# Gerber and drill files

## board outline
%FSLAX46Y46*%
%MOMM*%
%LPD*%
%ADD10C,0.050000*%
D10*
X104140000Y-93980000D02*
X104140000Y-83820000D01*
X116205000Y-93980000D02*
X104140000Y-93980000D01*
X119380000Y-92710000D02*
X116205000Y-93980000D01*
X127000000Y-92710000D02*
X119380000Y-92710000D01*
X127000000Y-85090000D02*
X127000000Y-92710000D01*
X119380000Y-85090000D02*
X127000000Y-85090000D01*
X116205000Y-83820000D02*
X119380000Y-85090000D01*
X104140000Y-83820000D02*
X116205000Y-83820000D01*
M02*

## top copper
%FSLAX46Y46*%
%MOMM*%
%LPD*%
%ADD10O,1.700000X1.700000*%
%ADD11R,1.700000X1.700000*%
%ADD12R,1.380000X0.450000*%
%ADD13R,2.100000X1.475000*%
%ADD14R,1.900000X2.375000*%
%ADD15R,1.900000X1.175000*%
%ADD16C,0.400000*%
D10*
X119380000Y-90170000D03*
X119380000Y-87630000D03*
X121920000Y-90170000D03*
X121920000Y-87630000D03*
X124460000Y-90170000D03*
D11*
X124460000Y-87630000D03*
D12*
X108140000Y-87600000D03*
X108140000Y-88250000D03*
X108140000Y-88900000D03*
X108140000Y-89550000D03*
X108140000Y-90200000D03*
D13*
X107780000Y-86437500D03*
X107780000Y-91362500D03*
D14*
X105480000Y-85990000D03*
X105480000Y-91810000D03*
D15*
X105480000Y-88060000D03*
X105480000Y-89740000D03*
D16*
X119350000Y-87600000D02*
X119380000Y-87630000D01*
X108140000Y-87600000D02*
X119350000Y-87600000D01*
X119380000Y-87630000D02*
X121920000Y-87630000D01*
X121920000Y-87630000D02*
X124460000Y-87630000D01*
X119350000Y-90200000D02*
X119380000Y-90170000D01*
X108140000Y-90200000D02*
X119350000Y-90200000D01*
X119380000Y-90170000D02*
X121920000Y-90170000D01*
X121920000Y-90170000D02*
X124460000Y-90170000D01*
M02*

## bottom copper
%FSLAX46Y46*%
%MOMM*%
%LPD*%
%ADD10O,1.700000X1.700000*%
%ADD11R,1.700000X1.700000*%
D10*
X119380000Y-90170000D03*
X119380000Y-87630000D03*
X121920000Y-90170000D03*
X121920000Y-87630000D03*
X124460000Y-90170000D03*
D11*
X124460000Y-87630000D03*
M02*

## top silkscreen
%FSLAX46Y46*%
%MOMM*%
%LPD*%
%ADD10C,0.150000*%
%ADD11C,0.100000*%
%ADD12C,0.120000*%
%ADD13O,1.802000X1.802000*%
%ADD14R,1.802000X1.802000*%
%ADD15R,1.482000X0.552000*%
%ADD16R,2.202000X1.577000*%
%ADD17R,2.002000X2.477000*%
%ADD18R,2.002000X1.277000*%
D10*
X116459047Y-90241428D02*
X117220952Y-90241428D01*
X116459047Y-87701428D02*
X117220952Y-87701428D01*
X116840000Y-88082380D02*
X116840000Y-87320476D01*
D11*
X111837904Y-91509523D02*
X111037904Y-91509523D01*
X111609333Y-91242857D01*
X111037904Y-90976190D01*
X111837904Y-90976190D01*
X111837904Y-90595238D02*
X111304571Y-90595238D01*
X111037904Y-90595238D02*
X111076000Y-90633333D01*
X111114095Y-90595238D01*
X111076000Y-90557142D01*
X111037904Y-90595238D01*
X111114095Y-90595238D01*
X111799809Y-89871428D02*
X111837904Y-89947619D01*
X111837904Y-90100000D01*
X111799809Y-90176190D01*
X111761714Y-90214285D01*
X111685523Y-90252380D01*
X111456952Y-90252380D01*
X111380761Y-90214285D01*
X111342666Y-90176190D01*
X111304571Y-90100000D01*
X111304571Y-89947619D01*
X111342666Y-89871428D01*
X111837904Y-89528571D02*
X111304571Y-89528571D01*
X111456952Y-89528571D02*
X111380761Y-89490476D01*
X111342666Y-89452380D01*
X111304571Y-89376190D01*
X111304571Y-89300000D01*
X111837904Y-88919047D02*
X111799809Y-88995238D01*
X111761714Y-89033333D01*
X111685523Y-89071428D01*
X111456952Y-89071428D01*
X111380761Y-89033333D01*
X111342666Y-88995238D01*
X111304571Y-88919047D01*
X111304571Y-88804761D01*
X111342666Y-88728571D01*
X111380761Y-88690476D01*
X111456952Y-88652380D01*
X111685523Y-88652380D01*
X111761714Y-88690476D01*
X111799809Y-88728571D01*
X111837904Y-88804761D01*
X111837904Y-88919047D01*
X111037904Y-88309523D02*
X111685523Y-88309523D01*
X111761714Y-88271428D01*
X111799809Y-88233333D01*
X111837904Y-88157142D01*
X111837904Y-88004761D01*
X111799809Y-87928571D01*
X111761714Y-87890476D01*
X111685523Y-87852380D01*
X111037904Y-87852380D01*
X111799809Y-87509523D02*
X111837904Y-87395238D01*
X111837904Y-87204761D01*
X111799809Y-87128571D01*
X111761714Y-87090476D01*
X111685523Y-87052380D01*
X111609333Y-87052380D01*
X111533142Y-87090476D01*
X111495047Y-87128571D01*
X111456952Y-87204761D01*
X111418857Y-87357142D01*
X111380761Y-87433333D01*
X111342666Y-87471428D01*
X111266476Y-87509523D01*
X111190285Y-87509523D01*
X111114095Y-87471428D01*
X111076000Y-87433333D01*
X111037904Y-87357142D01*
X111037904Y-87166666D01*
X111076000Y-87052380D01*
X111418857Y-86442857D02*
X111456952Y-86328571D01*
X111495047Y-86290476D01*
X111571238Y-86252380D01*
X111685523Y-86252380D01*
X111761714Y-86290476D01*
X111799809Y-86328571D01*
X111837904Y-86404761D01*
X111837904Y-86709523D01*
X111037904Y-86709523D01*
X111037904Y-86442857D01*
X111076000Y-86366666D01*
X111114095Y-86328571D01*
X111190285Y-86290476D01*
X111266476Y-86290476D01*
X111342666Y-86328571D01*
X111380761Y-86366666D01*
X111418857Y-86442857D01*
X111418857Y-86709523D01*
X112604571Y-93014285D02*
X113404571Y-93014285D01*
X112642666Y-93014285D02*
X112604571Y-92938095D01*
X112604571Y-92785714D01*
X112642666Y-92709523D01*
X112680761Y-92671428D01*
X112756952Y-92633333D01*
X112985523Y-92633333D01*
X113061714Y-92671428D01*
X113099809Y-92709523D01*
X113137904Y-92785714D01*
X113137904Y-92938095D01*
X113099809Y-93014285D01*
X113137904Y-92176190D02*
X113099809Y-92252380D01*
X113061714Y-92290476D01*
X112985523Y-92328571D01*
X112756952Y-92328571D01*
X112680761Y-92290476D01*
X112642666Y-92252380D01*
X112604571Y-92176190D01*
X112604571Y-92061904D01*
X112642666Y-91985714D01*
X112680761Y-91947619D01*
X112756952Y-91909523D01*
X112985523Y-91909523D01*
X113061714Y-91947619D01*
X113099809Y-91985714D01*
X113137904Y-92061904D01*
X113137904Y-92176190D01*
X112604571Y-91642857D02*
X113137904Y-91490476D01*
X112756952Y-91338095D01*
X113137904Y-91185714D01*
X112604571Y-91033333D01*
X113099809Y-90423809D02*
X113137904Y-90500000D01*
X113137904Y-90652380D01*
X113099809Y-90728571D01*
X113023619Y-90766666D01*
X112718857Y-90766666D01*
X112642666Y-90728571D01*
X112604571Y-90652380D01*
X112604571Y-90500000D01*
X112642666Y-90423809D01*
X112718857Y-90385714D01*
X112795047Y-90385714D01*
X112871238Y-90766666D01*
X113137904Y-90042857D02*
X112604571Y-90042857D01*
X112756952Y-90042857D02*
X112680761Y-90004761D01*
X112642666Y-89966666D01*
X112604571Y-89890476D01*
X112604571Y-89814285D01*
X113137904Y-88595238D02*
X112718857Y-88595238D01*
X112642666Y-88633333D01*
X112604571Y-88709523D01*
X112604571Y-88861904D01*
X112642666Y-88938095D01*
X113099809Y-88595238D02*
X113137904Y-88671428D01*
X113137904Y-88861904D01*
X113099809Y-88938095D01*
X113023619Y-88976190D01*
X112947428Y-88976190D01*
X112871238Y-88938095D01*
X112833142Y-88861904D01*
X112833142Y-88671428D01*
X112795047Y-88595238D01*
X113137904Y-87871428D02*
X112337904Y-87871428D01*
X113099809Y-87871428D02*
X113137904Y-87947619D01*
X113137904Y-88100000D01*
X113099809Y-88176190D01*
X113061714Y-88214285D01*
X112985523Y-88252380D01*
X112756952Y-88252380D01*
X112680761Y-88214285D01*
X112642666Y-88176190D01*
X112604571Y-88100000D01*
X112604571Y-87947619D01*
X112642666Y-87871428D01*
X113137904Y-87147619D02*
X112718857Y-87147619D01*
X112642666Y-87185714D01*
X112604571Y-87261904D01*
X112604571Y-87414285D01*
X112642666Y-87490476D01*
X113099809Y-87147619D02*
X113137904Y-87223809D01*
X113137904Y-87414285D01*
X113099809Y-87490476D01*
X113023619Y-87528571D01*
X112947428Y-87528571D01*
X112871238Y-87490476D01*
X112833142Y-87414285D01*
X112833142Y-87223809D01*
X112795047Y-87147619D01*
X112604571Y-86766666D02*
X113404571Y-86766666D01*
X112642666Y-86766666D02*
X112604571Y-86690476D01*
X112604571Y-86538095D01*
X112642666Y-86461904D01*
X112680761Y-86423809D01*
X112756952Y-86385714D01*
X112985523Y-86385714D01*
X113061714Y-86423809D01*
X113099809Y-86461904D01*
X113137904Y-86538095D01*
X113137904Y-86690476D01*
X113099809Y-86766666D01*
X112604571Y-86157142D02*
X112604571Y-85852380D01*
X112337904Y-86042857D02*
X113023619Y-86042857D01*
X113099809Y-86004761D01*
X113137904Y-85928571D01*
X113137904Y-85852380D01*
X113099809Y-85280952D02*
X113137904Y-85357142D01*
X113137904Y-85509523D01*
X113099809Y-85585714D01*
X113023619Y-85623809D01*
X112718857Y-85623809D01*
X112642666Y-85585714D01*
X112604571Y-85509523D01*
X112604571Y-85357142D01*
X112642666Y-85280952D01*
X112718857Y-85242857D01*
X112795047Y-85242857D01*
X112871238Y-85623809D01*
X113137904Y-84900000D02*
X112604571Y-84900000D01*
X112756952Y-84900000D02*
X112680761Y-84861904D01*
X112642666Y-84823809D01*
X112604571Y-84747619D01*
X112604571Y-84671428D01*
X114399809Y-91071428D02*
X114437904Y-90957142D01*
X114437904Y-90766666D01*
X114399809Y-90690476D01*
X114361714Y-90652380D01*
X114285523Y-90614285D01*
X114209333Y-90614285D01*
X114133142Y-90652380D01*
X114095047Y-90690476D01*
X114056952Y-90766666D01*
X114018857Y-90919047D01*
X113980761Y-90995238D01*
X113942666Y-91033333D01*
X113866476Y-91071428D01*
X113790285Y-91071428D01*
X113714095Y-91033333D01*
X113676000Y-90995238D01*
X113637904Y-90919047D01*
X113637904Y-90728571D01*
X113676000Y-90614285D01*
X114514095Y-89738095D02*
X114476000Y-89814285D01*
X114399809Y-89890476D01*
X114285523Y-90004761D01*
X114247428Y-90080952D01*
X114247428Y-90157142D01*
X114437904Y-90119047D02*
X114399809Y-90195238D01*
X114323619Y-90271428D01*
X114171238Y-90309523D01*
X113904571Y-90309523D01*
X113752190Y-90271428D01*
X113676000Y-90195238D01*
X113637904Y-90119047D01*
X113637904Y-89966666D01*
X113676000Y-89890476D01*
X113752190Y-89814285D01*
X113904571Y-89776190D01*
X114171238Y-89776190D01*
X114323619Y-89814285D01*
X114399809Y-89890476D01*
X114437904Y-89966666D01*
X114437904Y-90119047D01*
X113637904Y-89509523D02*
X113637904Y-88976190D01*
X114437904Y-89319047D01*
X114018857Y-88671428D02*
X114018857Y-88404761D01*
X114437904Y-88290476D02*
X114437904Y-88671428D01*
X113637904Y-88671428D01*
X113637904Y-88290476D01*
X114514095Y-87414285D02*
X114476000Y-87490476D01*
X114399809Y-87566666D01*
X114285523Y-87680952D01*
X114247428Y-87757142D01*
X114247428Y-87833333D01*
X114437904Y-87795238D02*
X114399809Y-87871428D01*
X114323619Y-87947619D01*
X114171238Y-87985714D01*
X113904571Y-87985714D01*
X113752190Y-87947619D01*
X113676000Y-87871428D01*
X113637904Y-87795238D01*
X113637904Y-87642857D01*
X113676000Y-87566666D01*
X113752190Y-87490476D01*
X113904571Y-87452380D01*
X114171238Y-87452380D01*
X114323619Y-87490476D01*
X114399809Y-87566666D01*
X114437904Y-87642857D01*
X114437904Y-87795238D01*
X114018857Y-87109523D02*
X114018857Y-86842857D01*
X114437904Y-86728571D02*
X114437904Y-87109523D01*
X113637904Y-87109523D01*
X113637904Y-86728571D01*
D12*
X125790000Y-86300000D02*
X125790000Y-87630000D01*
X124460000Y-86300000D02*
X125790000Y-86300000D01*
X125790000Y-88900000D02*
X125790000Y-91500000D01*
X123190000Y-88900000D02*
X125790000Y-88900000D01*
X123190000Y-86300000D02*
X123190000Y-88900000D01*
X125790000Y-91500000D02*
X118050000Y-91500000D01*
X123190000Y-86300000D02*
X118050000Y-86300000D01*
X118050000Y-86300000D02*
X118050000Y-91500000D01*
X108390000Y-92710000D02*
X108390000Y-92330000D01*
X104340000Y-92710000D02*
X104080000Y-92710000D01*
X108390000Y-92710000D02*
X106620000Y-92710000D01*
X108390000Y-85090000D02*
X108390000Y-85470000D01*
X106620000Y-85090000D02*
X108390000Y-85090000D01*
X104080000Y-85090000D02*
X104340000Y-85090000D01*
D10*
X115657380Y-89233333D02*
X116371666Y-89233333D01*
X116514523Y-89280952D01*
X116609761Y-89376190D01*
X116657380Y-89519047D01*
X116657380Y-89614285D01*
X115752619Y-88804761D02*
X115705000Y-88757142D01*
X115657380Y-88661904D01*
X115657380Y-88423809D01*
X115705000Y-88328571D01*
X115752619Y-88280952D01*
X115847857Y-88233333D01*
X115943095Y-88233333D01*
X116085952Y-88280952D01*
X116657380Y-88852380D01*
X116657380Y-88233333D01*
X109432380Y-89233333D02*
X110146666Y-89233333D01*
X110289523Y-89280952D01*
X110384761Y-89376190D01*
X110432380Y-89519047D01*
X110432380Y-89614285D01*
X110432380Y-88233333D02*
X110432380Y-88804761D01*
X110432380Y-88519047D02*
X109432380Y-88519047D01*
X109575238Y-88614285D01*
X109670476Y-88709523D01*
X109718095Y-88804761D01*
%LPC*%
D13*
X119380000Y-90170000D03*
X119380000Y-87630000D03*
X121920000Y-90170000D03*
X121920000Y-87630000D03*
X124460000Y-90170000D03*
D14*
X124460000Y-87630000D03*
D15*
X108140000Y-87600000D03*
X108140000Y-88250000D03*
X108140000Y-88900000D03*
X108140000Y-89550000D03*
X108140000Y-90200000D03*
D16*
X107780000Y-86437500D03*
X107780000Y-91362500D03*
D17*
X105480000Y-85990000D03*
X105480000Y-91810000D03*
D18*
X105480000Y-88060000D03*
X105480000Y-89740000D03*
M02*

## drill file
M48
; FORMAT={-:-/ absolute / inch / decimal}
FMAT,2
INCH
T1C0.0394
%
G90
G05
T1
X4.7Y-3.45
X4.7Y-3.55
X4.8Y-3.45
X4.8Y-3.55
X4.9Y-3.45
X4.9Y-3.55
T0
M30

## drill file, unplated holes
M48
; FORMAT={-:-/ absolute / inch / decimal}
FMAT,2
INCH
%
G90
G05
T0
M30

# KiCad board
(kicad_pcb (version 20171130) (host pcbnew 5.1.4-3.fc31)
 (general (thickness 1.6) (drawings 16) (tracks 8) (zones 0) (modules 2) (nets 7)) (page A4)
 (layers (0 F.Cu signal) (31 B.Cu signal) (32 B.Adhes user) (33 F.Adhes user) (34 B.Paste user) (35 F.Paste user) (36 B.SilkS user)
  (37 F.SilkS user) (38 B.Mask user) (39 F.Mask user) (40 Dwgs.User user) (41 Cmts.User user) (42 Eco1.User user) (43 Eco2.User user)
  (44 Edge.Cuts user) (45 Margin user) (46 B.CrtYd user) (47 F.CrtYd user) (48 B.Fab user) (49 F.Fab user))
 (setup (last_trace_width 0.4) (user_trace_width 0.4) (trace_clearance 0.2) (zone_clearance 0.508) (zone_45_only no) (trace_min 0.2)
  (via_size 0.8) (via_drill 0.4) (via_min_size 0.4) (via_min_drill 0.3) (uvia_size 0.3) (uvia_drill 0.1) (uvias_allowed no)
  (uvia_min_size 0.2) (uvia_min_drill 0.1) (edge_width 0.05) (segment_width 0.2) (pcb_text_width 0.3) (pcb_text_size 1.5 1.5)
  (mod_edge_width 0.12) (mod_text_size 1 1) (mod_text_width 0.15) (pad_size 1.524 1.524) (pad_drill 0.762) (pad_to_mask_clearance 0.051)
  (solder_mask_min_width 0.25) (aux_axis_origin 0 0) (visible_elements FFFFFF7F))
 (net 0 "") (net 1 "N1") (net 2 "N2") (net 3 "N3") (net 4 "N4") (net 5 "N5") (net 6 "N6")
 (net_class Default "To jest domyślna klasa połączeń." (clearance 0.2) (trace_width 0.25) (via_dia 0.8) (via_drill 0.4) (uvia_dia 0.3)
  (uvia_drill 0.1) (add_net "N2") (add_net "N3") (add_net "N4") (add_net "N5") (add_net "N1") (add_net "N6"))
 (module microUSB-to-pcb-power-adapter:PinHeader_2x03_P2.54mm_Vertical (layer F.Cu) (at 124.46 87.63 270)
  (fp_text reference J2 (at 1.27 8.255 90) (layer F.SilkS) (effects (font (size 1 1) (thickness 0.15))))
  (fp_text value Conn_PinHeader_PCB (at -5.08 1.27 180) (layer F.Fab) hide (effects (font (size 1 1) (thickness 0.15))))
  (fp_line (start -1.33 -1.33) (end 0 -1.33) (layer F.SilkS) (width 0.12))
  (fp_line (start -1.33 0) (end -1.33 -1.33) (layer F.SilkS) (width 0.12))
  (fp_line (start 1.27 -1.33) (end 3.87 -1.33) (layer F.SilkS) (width 0.12))
  (fp_line (start 1.27 1.27) (end 1.27 -1.33) (layer F.SilkS) (width 0.12))
  (fp_line (start -1.33 1.27) (end 1.27 1.27) (layer F.SilkS) (width 0.12))
  (fp_line (start 3.87 -1.33) (end 3.87 6.41) (layer F.SilkS) (width 0.12))
  (fp_line (start -1.33 1.27) (end -1.33 6.41) (layer F.SilkS) (width 0.12))
  (fp_line (start -1.33 6.41) (end 3.87 6.41) (layer F.SilkS) (width 0.12))
  (pad 4 thru_hole oval (at 2.54 5.08 270) (size 1.7 1.7) (drill 1) (layers *.Cu *.Mask) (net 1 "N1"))
  (pad 3 thru_hole oval (at 0 5.08 270) (size 1.7 1.7) (drill 1) (layers *.Cu *.Mask) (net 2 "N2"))
  (pad 5 thru_hole oval (at 2.54 2.54 270) (size 1.7 1.7) (drill 1) (layers *.Cu *.Mask) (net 1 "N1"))
  (pad 2 thru_hole oval (at 0 2.54 270) (size 1.7 1.7) (drill 1) (layers *.Cu *.Mask) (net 2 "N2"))
  (pad 6 thru_hole oval (at 2.54 0 270) (size 1.7 1.7) (drill 1) (layers *.Cu *.Mask) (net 1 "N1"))
  (pad 1 thru_hole rect (at 0 0 270) (size 1.7 1.7) (drill 1) (layers *.Cu *.Mask) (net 2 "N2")))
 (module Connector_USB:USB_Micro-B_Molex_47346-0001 (layer F.Cu) (at 106.68 88.9 270)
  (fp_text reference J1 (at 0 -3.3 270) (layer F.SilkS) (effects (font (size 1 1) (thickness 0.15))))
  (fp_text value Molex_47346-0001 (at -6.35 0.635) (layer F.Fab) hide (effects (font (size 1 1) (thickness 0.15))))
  (fp_line (start 3.81 -1.71) (end 3.43 -1.71) (layer F.SilkS) (width 0.12))
  (fp_line (start 3.81 2.34) (end 3.81 2.6) (layer F.SilkS) (width 0.12))
  (fp_line (start 3.81 -1.71) (end 3.81 0.06) (layer F.SilkS) (width 0.12))
  (fp_line (start -3.81 -1.71) (end -3.43 -1.71) (layer F.SilkS) (width 0.12))
  (fp_line (start -3.81 0.06) (end -3.81 -1.71) (layer F.SilkS) (width 0.12))
  (fp_line (start -3.81 2.6) (end -3.81 2.34) (layer F.SilkS) (width 0.12))
  (pad 1 smd rect (at -1.3 -1.46 270) (size 0.45 1.38) (layers F.Cu F.Paste F.Mask) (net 2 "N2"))
  (pad 2 smd rect (at -0.65 -1.46 270) (size 0.45 1.38) (layers F.Cu F.Paste F.Mask) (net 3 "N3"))
  (pad 3 smd rect (at 0 -1.46 270) (size 0.45 1.38) (layers F.Cu F.Paste F.Mask) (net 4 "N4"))
  (pad 4 smd rect (at 0.65 -1.46 270) (size 0.45 1.38) (layers F.Cu F.Paste F.Mask) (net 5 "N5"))
  (pad 5 smd rect (at 1.3 -1.46 270) (size 0.45 1.38) (layers F.Cu F.Paste F.Mask) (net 1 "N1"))
  (pad 6 smd rect (at -2.4625 -1.1 270) (size 1.475 2.1) (layers F.Cu F.Paste F.Mask) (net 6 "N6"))
  (pad 6 smd rect (at 2.4625 -1.1 270) (size 1.475 2.1) (layers F.Cu F.Paste F.Mask) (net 6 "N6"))
  (pad 6 smd rect (at -2.91 1.2 270) (size 2.375 1.9) (layers F.Cu F.Paste F.Mask) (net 6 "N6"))
  (pad 6 smd rect (at 2.91 1.2 270) (size 2.375 1.9) (layers F.Cu F.Paste F.Mask) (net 6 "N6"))
  (pad 6 smd rect (at -0.84 1.2 270) (size 1.175 1.9) (layers F.Cu F.Paste F.Mask) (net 6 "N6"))
  (pad 6 smd rect (at 0.84 1.2 270) (size 1.175 1.9) (layers F.Cu F.Paste F.Mask) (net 6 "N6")))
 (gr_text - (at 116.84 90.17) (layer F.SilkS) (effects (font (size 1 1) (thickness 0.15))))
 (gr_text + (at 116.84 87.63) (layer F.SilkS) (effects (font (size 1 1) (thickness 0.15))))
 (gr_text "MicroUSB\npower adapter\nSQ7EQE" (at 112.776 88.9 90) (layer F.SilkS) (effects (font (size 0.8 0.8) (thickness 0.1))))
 (gr_line (start 104.14 93.98) (end 104.14 83.82) (layer Edge.Cuts) (width 0.05))
 (gr_line (start 116.205 93.98) (end 104.14 93.98) (layer Edge.Cuts) (width 0.05))
 (gr_line (start 119.38 92.71) (end 116.205 93.98) (layer Edge.Cuts) (width 0.05))
 (gr_line (start 127 92.71) (end 119.38 92.71) (layer Edge.Cuts) (width 0.05))
 (gr_line (start 127 85.09) (end 127 92.71) (layer Edge.Cuts) (width 0.05))
 (gr_line (start 119.38 85.09) (end 127 85.09) (layer Edge.Cuts) (width 0.05))
 (gr_line (start 116.205 83.82) (end 119.38 85.09) (layer Edge.Cuts) (width 0.05))
 (gr_line (start 104.14 83.82) (end 116.205 83.82) (layer Edge.Cuts) (width 0.05))
 (segment (start 119.35 87.6) (end 119.38 87.63) (width 0.4) (layer F.Cu) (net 2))
 (segment (start 108.14 87.6) (end 119.35 87.6) (width 0.4) (layer F.Cu) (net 2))
 (segment (start 119.38 87.63) (end 121.92 87.63) (width 0.4) (layer F.Cu) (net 2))
 (segment (start 121.92 87.63) (end 124.46 87.63) (width 0.4) (layer F.Cu) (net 2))
 (segment (start 119.35 90.2) (end 119.38 90.17) (width 0.4) (layer F.Cu) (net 1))
 (segment (start 108.14 90.2) (end 119.35 90.2) (width 0.4) (layer F.Cu) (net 1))
 (segment (start 119.38 90.17) (end 121.92 90.17) (width 0.4) (layer F.Cu) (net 1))
 (segment (start 121.92 90.17) (end 124.46 90.17) (width 0.4) (layer F.Cu) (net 1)))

